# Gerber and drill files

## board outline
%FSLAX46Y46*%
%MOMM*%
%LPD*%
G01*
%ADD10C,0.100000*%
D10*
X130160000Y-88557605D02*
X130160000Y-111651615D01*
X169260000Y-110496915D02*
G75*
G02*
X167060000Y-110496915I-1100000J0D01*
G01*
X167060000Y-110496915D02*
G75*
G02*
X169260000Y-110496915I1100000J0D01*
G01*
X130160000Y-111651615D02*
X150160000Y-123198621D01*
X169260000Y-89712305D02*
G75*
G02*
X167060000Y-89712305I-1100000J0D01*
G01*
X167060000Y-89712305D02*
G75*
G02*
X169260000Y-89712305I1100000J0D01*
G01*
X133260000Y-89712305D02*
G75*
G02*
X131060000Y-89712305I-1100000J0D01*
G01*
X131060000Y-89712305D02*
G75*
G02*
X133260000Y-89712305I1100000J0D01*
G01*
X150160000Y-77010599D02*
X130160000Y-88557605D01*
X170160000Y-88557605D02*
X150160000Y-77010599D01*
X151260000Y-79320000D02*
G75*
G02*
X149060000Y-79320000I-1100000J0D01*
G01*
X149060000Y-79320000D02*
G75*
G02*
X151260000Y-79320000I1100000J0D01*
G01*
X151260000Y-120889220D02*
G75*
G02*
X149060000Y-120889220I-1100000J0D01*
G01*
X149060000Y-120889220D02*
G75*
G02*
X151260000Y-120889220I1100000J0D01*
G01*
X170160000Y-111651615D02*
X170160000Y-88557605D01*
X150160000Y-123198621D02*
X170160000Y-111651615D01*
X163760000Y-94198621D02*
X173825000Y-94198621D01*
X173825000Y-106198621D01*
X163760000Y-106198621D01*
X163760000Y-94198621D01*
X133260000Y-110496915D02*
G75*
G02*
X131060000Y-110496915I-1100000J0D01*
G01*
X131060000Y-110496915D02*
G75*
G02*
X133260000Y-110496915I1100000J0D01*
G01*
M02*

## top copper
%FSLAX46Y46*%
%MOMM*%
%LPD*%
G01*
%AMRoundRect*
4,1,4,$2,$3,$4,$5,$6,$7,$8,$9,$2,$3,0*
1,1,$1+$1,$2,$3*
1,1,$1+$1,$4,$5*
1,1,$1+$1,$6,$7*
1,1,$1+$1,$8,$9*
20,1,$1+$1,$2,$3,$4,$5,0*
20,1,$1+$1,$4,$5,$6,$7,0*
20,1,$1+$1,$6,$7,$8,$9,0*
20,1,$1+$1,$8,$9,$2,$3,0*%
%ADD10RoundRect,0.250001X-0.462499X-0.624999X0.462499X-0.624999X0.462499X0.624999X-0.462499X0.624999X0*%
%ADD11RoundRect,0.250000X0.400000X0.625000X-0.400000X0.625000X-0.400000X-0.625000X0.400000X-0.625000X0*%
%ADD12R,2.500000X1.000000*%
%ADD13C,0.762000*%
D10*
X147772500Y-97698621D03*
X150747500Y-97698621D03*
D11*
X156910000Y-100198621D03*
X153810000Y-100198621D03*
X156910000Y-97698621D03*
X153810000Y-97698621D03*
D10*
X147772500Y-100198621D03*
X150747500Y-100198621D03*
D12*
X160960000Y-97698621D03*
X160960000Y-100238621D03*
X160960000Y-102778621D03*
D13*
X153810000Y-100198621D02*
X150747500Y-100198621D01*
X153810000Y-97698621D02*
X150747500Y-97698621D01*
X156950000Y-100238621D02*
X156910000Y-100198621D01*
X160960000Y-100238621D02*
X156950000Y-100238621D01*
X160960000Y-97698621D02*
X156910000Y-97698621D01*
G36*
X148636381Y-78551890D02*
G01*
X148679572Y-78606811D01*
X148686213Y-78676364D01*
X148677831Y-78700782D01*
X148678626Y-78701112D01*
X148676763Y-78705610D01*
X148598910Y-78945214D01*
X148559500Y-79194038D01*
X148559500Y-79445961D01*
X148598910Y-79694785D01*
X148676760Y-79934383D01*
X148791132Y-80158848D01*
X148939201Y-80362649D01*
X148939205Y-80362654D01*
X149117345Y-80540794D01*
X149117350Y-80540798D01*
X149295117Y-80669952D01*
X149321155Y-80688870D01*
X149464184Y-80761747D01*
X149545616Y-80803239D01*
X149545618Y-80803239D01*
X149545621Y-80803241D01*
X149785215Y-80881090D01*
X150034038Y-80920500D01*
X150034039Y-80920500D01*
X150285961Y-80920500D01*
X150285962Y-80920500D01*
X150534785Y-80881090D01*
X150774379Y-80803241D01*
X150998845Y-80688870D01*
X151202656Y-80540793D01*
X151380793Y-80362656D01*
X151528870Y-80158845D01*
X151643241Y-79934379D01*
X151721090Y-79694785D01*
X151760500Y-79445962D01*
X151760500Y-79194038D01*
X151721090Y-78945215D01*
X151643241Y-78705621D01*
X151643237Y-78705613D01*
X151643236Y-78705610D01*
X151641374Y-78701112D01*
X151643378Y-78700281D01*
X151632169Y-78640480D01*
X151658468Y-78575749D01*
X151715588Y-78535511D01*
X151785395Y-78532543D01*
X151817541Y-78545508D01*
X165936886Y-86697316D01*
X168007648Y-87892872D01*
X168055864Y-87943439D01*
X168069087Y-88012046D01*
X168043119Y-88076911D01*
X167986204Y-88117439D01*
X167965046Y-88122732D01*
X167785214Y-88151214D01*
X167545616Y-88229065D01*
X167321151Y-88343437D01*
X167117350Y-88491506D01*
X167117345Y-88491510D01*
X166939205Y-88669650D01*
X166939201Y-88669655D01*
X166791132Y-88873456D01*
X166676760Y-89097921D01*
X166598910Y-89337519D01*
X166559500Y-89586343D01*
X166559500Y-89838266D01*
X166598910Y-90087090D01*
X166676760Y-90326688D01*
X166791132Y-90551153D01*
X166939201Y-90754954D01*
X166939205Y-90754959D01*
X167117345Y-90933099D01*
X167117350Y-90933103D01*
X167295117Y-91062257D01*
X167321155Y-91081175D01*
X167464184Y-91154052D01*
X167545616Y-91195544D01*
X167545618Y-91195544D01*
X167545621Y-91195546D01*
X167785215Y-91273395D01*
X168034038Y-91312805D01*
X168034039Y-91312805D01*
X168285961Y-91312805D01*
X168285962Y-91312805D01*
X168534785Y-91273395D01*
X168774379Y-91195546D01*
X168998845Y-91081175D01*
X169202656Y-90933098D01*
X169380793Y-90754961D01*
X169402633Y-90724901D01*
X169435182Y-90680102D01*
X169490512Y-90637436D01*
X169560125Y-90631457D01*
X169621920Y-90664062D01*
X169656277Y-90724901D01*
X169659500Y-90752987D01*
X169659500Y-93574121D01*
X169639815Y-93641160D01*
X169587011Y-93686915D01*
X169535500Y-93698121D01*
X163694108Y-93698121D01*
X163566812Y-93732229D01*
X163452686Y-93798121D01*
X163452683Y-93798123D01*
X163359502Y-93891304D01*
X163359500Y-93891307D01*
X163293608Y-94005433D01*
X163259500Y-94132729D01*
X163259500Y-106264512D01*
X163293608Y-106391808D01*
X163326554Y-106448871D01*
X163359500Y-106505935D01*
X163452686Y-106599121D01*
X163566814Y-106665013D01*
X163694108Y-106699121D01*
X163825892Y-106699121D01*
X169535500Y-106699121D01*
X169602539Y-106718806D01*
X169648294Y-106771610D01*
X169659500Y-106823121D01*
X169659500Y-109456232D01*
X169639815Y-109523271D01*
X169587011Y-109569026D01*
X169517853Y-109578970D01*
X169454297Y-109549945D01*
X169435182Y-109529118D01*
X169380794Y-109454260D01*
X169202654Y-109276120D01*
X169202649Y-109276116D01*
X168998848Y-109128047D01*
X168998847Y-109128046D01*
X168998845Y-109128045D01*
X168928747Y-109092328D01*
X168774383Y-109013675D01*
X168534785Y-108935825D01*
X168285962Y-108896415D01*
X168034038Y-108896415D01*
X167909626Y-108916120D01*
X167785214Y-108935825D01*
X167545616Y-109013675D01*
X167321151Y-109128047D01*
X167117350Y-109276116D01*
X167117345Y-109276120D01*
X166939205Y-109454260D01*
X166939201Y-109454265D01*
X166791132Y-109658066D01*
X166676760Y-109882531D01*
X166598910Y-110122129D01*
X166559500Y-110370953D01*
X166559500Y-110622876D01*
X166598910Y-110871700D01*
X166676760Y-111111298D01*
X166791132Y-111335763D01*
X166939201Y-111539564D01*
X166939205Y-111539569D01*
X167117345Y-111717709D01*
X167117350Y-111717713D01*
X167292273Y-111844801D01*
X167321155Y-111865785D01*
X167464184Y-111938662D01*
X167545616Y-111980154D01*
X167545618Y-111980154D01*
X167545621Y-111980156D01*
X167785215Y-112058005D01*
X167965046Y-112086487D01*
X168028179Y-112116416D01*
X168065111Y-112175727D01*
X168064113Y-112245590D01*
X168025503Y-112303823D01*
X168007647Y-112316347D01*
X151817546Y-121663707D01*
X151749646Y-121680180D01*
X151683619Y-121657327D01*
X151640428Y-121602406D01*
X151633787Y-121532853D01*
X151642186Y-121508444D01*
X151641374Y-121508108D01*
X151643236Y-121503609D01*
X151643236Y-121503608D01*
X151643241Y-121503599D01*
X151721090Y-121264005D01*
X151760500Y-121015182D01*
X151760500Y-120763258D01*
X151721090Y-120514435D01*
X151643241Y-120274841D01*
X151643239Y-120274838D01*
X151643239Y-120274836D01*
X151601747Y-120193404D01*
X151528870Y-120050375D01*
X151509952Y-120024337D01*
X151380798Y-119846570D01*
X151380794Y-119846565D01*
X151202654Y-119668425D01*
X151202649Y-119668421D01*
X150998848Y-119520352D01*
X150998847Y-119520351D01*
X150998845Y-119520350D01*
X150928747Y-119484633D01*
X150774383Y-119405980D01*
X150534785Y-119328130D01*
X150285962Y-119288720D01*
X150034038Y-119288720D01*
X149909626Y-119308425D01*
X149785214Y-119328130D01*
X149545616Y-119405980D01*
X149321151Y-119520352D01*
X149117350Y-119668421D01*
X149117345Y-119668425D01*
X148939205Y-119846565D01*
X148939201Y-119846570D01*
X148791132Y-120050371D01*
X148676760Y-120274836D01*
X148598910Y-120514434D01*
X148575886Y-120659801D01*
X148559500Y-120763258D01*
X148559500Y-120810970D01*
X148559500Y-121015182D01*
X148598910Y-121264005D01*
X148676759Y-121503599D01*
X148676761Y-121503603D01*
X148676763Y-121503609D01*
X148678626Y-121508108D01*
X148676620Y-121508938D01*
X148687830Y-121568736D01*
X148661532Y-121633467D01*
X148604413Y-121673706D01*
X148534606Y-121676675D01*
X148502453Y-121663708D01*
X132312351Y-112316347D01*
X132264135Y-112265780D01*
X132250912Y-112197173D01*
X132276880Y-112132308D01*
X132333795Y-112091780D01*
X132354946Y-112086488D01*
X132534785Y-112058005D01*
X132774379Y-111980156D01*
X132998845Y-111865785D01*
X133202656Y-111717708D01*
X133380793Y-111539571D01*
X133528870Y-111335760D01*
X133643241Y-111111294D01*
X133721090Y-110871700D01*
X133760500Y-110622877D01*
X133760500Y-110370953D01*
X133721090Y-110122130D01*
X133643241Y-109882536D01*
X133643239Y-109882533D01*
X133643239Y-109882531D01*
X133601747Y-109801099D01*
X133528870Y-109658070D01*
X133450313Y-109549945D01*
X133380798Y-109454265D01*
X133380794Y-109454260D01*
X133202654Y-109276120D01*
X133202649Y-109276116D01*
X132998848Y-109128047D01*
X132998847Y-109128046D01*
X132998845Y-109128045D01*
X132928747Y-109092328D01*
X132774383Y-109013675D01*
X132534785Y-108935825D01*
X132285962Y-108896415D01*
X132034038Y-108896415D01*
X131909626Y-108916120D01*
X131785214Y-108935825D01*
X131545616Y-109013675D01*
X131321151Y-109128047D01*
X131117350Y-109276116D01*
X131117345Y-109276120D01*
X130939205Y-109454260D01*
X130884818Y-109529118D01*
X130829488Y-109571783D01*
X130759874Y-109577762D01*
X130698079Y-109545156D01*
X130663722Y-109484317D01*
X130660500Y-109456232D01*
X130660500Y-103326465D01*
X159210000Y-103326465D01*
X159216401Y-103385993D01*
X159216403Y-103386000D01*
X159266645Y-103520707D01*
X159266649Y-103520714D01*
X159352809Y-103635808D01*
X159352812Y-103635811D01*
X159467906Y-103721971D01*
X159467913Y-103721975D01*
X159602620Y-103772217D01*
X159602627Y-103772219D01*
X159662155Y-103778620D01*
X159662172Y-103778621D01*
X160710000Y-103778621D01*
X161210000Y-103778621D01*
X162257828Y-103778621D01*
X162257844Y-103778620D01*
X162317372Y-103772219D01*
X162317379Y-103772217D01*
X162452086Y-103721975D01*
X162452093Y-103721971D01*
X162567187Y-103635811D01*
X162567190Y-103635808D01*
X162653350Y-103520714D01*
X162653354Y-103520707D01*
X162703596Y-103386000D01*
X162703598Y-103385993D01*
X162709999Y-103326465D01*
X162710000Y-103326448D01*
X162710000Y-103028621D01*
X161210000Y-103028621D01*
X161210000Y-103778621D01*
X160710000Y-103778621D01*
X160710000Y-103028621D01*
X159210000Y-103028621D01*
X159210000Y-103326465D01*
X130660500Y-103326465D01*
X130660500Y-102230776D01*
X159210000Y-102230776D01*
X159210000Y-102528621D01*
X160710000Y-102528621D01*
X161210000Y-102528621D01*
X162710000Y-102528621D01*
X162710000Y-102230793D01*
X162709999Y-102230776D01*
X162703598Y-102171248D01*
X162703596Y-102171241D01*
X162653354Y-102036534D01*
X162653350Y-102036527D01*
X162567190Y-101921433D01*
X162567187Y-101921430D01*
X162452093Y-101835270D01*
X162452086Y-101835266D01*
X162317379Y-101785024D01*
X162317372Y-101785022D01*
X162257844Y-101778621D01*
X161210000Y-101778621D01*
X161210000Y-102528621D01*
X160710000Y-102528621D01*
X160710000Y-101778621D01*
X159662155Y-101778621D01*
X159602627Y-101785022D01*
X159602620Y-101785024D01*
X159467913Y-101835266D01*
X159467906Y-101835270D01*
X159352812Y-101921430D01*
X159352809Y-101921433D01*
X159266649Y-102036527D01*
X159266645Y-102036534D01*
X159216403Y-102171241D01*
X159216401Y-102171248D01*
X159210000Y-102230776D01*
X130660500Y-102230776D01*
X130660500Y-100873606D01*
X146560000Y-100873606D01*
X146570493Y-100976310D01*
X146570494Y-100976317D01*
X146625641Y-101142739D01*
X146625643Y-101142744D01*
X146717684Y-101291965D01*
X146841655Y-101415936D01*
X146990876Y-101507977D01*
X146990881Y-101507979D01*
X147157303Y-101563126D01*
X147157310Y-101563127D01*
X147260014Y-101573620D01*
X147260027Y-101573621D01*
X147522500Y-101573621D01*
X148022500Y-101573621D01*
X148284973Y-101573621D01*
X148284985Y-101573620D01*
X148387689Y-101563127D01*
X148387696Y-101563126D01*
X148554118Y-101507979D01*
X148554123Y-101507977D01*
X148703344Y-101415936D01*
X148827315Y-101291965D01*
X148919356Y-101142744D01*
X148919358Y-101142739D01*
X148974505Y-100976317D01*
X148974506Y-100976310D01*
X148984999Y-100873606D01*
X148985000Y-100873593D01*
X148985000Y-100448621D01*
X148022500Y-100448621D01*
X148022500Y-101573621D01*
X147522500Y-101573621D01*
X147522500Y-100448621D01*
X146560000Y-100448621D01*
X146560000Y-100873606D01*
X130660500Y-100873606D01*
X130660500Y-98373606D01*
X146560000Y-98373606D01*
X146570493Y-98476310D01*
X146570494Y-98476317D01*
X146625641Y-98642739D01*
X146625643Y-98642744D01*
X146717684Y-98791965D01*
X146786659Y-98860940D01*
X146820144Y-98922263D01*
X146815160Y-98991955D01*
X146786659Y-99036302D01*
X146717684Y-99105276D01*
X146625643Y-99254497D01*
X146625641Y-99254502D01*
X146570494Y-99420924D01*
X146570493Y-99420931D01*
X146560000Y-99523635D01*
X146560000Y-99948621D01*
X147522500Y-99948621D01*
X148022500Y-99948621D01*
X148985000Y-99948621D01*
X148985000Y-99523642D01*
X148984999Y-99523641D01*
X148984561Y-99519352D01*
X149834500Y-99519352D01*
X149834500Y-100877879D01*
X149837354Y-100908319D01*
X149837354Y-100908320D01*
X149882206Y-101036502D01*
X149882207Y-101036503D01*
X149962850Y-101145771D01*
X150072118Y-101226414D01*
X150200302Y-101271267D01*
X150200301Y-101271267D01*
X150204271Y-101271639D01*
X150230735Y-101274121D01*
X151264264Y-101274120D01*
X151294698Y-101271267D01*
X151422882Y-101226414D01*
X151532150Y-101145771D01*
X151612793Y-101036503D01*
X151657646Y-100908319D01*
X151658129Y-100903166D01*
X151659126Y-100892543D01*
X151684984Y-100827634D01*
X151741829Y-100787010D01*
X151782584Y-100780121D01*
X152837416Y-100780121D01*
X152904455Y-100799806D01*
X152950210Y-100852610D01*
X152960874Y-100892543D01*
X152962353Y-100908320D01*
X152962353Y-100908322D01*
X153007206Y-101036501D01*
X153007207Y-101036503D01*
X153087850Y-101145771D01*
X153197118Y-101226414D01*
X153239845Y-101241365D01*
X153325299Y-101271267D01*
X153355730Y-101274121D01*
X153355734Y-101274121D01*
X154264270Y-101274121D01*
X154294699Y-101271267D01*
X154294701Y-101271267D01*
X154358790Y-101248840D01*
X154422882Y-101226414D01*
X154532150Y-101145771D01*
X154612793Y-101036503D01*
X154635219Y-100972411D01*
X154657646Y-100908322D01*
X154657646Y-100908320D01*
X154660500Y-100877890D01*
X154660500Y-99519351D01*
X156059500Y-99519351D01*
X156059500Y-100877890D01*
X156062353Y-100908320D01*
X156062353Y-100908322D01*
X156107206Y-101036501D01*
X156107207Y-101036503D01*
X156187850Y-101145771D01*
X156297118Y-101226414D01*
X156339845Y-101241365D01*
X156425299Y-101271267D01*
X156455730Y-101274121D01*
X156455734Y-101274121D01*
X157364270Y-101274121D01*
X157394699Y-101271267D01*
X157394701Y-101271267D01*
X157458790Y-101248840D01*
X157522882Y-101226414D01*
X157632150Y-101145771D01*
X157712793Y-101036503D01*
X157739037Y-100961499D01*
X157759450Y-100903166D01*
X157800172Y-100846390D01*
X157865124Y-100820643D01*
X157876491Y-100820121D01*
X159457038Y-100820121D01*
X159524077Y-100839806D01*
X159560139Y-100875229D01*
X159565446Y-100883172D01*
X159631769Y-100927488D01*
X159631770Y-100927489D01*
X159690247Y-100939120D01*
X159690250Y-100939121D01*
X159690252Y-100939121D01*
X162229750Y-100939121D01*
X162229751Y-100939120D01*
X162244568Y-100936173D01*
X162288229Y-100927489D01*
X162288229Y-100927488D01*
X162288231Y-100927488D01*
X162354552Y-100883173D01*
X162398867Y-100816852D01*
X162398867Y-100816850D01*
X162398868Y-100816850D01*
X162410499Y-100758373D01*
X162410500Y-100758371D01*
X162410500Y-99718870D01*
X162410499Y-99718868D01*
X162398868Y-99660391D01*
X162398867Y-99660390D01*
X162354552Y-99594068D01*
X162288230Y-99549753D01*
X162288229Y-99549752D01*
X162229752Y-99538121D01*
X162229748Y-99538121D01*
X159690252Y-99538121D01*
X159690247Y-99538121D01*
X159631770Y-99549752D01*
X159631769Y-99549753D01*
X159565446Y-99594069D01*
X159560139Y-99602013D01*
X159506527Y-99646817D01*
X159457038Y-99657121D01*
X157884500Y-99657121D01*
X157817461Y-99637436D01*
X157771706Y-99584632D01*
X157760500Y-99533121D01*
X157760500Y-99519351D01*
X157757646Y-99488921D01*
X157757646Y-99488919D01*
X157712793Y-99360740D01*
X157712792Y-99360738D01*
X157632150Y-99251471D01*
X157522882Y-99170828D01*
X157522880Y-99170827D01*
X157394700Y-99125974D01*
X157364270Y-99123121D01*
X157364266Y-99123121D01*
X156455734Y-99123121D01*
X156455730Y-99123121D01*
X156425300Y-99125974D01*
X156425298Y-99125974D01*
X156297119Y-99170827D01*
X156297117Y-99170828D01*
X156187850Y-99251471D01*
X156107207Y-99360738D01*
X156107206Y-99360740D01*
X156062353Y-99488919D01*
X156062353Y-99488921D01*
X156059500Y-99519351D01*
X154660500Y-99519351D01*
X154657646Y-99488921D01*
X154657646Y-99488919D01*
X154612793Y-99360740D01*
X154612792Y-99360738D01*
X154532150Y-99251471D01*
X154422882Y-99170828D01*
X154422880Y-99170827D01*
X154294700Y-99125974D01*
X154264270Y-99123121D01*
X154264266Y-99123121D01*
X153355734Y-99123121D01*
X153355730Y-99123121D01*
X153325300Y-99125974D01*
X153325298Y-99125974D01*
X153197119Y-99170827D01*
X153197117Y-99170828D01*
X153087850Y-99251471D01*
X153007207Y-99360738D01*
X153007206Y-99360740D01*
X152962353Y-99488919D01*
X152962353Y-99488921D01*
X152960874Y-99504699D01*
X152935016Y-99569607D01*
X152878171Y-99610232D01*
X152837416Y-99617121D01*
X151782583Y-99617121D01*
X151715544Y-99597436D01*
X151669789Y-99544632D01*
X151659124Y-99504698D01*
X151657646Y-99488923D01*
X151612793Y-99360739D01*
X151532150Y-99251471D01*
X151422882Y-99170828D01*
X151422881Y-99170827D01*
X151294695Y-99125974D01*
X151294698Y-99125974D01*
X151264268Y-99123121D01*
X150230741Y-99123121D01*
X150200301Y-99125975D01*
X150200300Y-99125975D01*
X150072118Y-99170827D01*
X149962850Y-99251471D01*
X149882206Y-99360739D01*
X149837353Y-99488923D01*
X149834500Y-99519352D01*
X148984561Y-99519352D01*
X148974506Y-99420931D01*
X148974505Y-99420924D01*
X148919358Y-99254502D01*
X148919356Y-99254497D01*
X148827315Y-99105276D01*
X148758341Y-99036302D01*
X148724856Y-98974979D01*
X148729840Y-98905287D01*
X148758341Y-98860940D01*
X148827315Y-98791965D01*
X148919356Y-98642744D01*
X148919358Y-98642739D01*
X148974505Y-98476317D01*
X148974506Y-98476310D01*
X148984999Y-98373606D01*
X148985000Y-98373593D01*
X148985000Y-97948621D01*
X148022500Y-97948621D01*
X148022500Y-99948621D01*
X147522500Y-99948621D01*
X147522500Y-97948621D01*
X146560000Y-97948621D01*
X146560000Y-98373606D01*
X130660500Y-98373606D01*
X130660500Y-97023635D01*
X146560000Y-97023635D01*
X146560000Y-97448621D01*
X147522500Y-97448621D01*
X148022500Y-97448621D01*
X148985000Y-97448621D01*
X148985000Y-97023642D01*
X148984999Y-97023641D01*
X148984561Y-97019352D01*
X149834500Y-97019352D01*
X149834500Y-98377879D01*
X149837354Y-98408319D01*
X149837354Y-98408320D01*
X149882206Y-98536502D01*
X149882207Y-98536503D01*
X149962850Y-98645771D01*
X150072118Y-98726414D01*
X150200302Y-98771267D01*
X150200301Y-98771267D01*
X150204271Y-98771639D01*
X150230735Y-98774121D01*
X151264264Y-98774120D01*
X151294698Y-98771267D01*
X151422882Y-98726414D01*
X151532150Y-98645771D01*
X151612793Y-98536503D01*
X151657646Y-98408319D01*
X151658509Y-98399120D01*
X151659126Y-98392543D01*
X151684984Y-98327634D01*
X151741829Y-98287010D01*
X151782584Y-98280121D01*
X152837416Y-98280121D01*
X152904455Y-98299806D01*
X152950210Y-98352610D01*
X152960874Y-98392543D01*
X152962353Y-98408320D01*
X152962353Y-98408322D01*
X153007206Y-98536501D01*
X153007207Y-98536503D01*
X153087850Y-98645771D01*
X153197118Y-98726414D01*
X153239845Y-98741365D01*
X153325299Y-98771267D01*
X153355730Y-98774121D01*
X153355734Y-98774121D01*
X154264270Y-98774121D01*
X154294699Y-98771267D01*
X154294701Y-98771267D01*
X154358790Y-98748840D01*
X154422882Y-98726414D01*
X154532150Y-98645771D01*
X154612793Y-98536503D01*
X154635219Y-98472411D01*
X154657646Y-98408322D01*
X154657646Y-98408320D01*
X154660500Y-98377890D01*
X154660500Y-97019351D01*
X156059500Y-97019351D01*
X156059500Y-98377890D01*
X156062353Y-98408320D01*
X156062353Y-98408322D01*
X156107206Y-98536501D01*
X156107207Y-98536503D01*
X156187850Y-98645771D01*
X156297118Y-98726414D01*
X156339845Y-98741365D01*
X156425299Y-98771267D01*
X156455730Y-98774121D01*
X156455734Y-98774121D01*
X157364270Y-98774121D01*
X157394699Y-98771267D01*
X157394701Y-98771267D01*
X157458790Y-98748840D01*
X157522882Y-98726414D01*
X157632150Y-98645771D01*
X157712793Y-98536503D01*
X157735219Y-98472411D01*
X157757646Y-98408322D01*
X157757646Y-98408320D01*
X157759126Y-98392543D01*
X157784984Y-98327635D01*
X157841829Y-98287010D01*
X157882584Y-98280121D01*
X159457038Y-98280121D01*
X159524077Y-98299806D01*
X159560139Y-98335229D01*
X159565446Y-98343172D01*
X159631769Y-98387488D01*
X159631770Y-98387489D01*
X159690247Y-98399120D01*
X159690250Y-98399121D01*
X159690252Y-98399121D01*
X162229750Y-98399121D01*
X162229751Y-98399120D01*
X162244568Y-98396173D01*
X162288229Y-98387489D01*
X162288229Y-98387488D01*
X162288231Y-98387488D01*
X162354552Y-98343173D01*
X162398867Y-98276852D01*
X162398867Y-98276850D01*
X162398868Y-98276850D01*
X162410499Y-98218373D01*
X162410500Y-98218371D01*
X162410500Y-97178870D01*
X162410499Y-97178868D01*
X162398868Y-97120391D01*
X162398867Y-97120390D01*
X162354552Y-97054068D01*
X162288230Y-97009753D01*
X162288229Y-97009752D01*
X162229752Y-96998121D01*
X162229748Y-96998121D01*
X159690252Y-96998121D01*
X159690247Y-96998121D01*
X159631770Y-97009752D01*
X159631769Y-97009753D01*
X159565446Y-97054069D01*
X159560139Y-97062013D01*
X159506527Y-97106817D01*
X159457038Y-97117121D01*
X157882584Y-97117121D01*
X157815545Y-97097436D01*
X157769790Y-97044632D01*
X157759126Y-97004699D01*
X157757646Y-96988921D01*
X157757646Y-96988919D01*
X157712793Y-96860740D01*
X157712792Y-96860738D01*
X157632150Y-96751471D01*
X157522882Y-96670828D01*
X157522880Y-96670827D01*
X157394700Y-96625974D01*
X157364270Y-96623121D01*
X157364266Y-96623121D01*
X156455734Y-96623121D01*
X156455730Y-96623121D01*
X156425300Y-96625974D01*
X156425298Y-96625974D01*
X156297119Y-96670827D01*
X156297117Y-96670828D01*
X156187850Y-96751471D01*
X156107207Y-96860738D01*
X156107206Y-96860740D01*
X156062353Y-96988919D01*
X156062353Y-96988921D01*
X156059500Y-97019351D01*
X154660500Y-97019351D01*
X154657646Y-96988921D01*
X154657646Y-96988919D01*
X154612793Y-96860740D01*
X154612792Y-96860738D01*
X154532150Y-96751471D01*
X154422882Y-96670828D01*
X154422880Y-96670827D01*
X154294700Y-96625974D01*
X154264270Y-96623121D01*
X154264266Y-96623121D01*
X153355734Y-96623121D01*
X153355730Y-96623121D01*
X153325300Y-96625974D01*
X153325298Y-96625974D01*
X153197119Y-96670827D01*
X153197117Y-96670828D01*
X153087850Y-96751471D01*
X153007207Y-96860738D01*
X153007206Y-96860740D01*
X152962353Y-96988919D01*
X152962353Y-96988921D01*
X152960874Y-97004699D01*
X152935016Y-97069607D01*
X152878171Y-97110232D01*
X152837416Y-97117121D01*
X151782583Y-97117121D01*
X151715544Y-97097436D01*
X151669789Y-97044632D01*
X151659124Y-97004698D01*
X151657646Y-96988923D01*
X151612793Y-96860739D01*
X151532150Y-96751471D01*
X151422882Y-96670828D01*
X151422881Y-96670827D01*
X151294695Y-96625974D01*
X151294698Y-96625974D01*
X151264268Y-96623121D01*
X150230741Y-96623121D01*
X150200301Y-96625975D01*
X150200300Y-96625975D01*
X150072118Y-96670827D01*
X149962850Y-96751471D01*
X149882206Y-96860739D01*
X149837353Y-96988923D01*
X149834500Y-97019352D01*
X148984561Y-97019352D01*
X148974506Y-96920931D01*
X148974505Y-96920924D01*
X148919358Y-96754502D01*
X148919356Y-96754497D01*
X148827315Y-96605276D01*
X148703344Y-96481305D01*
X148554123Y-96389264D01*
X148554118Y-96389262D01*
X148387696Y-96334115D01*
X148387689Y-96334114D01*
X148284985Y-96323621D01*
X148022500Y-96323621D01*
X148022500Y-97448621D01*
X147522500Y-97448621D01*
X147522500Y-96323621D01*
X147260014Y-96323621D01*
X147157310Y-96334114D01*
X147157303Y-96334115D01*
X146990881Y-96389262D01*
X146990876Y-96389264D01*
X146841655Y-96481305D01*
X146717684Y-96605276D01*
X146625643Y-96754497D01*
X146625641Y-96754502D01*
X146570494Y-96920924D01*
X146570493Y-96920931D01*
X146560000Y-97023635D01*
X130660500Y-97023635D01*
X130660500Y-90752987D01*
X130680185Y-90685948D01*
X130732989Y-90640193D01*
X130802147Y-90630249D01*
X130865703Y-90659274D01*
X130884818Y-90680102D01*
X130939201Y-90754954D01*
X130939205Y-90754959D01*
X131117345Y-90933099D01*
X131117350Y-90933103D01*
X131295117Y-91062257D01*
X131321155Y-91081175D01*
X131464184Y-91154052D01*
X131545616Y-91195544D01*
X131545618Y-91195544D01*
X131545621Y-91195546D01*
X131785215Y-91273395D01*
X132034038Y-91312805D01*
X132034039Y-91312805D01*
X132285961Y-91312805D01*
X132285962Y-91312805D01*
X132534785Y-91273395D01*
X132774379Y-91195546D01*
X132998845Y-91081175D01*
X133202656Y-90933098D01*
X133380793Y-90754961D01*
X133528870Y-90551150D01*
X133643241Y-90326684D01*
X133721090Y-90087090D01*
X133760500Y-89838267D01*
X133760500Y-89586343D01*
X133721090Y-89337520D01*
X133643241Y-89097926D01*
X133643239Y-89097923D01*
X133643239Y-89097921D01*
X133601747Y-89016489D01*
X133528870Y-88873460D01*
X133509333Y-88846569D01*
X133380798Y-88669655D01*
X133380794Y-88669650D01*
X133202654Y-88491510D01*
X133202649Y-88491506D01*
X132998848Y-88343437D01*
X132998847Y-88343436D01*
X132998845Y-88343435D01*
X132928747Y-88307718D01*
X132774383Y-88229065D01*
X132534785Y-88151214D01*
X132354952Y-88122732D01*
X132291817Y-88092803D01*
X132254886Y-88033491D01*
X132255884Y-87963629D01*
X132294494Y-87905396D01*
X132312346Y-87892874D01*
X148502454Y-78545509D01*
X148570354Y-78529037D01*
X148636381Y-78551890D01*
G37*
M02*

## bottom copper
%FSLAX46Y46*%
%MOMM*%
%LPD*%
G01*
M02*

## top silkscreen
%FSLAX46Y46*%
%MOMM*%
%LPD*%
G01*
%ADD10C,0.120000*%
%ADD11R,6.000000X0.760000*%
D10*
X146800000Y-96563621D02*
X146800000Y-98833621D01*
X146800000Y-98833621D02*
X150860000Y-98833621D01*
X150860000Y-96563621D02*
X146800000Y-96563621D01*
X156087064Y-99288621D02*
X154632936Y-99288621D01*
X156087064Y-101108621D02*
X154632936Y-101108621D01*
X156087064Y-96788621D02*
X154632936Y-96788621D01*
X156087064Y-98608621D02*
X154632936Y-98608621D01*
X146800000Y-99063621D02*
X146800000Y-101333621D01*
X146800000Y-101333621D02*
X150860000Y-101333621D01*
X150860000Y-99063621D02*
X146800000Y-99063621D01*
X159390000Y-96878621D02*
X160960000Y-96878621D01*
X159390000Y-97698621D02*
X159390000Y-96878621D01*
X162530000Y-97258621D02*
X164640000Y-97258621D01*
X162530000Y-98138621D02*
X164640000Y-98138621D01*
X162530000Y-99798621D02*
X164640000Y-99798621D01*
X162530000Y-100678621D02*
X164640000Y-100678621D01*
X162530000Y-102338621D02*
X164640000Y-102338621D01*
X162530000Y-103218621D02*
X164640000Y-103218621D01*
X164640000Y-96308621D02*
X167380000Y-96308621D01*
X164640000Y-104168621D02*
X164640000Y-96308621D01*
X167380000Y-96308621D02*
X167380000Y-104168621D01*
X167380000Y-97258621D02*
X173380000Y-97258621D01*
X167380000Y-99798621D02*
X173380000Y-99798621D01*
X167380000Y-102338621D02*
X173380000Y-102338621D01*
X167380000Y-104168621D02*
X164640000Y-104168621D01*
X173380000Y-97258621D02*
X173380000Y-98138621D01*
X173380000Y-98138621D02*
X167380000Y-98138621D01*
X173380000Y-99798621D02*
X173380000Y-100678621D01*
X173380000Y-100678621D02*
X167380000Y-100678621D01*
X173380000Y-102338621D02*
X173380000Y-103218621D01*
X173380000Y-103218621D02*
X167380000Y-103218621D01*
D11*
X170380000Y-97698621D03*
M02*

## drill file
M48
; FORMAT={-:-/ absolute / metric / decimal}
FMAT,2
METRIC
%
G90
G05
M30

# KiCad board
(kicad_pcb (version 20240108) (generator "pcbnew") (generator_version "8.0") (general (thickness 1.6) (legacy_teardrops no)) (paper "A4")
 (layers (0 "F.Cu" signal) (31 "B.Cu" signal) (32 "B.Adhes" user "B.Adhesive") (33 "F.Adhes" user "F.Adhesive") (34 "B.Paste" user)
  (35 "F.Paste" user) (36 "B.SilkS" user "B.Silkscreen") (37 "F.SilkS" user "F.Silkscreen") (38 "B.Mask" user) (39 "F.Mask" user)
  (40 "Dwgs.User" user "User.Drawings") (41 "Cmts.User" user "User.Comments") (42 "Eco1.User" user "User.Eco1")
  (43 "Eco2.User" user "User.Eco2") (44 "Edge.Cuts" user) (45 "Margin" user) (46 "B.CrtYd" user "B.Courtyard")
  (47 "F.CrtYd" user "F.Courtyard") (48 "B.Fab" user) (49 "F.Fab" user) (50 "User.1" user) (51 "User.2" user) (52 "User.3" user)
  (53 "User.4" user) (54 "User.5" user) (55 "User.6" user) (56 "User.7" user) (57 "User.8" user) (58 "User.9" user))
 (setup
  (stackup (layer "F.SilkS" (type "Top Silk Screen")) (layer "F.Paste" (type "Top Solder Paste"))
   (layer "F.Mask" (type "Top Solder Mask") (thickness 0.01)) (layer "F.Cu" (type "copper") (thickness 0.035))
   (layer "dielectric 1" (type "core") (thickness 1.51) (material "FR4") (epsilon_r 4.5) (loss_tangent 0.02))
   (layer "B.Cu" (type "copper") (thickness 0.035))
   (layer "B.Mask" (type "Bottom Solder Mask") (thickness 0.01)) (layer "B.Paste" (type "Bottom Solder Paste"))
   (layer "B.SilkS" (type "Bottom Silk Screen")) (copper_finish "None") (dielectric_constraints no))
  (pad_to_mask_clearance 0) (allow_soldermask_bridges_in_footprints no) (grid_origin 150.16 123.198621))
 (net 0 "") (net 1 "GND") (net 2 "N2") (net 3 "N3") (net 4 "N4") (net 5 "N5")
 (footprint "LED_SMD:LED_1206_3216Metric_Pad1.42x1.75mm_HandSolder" (layer "F.Cu") (at 149.26 97.698621)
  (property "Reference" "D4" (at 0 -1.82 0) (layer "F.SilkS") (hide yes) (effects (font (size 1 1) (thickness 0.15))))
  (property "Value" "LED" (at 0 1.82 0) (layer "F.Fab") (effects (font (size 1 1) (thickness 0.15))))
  (fp_line (start -2.46 -1.135) (end -2.46 1.135) (stroke (width 0.12) (type solid)) (layer "F.SilkS"))
  (fp_line (start -2.46 1.135) (end 1.6 1.135) (stroke (width 0.12) (type solid)) (layer "F.SilkS"))
  (fp_line (start 1.6 -1.135) (end -2.46 -1.135) (stroke (width 0.12) (type solid)) (layer "F.SilkS"))
  (pad "1" smd roundrect (at -1.4875 0) (size 1.425 1.75) (layers "F.Cu" "F.Paste" "F.Mask") (roundrect_rratio 0.175439) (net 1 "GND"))
  (pad "2" smd roundrect (at 1.4875 0) (size 1.425 1.75) (layers "F.Cu" "F.Paste" "F.Mask") (roundrect_rratio 0.175439) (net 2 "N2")))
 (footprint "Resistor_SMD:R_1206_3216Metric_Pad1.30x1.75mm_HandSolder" (layer "F.Cu") (at 155.36 100.198621 180)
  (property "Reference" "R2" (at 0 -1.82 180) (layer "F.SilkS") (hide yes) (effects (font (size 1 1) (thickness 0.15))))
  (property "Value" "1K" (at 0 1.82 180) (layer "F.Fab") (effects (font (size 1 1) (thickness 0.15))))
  (fp_line (start -0.727064 0.91) (end 0.727064 0.91) (stroke (width 0.12) (type solid)) (layer "F.SilkS"))
  (fp_line (start -0.727064 -0.91) (end 0.727064 -0.91) (stroke (width 0.12) (type solid)) (layer "F.SilkS"))
  (pad "1" smd roundrect (at -1.55 0 180) (size 1.3 1.75) (layers "F.Cu" "F.Paste" "F.Mask") (roundrect_rratio 0.192308) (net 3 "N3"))
  (pad "2" smd roundrect (at 1.55 0 180) (size 1.3 1.75) (layers "F.Cu" "F.Paste" "F.Mask") (roundrect_rratio 0.192308) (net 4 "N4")))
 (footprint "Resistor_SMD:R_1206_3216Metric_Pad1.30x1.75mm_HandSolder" (layer "F.Cu") (at 155.36 97.698621 180)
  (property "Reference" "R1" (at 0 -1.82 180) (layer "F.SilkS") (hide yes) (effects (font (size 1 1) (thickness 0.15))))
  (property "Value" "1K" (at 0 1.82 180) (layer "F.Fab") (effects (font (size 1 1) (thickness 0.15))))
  (fp_line (start -0.727064 0.91) (end 0.727064 0.91) (stroke (width 0.12) (type solid)) (layer "F.SilkS"))
  (fp_line (start -0.727064 -0.91) (end 0.727064 -0.91) (stroke (width 0.12) (type solid)) (layer "F.SilkS"))
  (pad "1" smd roundrect (at -1.55 0 180) (size 1.3 1.75) (layers "F.Cu" "F.Paste" "F.Mask") (roundrect_rratio 0.192308) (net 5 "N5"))
  (pad "2" smd roundrect (at 1.55 0 180) (size 1.3 1.75) (layers "F.Cu" "F.Paste" "F.Mask") (roundrect_rratio 0.192308) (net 2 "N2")))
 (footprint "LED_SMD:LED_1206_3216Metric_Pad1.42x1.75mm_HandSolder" (layer "F.Cu") (at 149.26 100.198621)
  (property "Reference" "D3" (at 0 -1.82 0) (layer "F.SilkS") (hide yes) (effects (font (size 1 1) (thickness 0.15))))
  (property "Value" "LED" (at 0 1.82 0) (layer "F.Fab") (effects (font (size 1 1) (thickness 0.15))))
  (fp_line (start -2.46 -1.135) (end -2.46 1.135) (stroke (width 0.12) (type solid)) (layer "F.SilkS"))
  (fp_line (start -2.46 1.135) (end 1.6 1.135) (stroke (width 0.12) (type solid)) (layer "F.SilkS"))
  (fp_line (start 1.6 -1.135) (end -2.46 -1.135) (stroke (width 0.12) (type solid)) (layer "F.SilkS"))
  (pad "1" smd roundrect (at -1.4875 0) (size 1.425 1.75) (layers "F.Cu" "F.Paste" "F.Mask") (roundrect_rratio 0.175439) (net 1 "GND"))
  (pad "2" smd roundrect (at 1.4875 0) (size 1.425 1.75) (layers "F.Cu" "F.Paste" "F.Mask") (roundrect_rratio 0.175439) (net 4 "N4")))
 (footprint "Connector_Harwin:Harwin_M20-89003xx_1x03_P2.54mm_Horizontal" (layer "F.Cu") (at 166.485 100.238621)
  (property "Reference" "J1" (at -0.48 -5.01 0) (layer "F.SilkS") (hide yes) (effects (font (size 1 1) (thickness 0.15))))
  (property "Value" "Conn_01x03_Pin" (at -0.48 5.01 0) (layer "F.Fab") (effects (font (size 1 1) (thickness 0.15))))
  (fp_line (start -7.095 -3.36) (end -5.525 -3.36) (stroke (width 0.12) (type solid)) (layer "F.SilkS"))
  (fp_line (start -7.095 -2.54) (end -7.095 -3.36) (stroke (width 0.12) (type solid)) (layer "F.SilkS"))
  (fp_line (start -3.955 -2.98) (end -1.845 -2.98) (stroke (width 0.12) (type solid)) (layer "F.SilkS"))
  (fp_line (start -3.955 -2.1) (end -1.845 -2.1) (stroke (width 0.12) (type solid)) (layer "F.SilkS"))
  (fp_line (start -3.955 -0.44) (end -1.845 -0.44) (stroke (width 0.12) (type solid)) (layer "F.SilkS"))
  (fp_line (start -3.955 0.44) (end -1.845 0.44) (stroke (width 0.12) (type solid)) (layer "F.SilkS"))
  (fp_line (start -3.955 2.1) (end -1.845 2.1) (stroke (width 0.12) (type solid)) (layer "F.SilkS"))
  (fp_line (start -3.955 2.98) (end -1.845 2.98) (stroke (width 0.12) (type solid)) (layer "F.SilkS"))
  (fp_line (start -1.845 -3.93) (end 0.895 -3.93) (stroke (width 0.12) (type solid)) (layer "F.SilkS"))
  (fp_line (start -1.845 3.93) (end -1.845 -3.93) (stroke (width 0.12) (type solid)) (layer "F.SilkS"))
  (fp_line (start 0.895 -3.93) (end 0.895 3.93) (stroke (width 0.12) (type solid)) (layer "F.SilkS"))
  (fp_line (start 0.895 -2.98) (end 6.895 -2.98) (stroke (width 0.12) (type solid)) (layer "F.SilkS"))
  (fp_line (start 0.895 -0.44) (end 6.895 -0.44) (stroke (width 0.12) (type solid)) (layer "F.SilkS"))
  (fp_line (start 0.895 2.1) (end 6.895 2.1) (stroke (width 0.12) (type solid)) (layer "F.SilkS"))
  (fp_line (start 0.895 3.93) (end -1.845 3.93) (stroke (width 0.12) (type solid)) (layer "F.SilkS"))
  (fp_line (start 6.895 -2.98) (end 6.895 -2.1) (stroke (width 0.12) (type solid)) (layer "F.SilkS"))
  (fp_line (start 6.895 -2.1) (end 0.895 -2.1) (stroke (width 0.12) (type solid)) (layer "F.SilkS"))
  (fp_line (start 6.895 -0.44) (end 6.895 0.44) (stroke (width 0.12) (type solid)) (layer "F.SilkS"))
  (fp_line (start 6.895 0.44) (end 0.895 0.44) (stroke (width 0.12) (type solid)) (layer "F.SilkS"))
  (fp_line (start 6.895 2.1) (end 6.895 2.98) (stroke (width 0.12) (type solid)) (layer "F.SilkS"))
  (fp_line (start 6.895 2.98) (end 0.895 2.98) (stroke (width 0.12) (type solid)) (layer "F.SilkS"))
  (pad "" smd rect (at 3.895 -2.54) (size 6 0.76) (layers "F.SilkS"))
  (pad "1" smd rect (at -5.525 -2.54) (size 2.5 1) (layers "F.Cu" "F.Paste" "F.Mask") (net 5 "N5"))
  (pad "2" smd rect (at -5.525 0) (size 2.5 1) (layers "F.Cu" "F.Paste" "F.Mask") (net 3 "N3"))
  (pad "3" smd rect (at -5.525 2.54) (size 2.5 1) (layers "F.Cu" "F.Paste" "F.Mask") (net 1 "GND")))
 (gr_line (start 130.16 88.557605) (end 130.16 111.651615) (stroke (width 0.1) (type solid)) (layer "Edge.Cuts"))
 (gr_circle (center 168.16 110.496915) (end 169.26 110.496915) (stroke (width 0.1) (type solid)) (fill none) (layer "Edge.Cuts"))
 (gr_line (start 130.16 111.651615) (end 150.16 123.198621) (stroke (width 0.1) (type solid)) (layer "Edge.Cuts"))
 (gr_circle (center 168.16 89.712305) (end 169.26 89.712305) (stroke (width 0.1) (type solid)) (fill none) (layer "Edge.Cuts"))
 (gr_circle (center 132.16 89.712305) (end 133.26 89.712305) (stroke (width 0.1) (type solid)) (fill none) (layer "Edge.Cuts"))
 (gr_line (start 150.16 77.010599) (end 130.16 88.557605) (stroke (width 0.1) (type solid)) (layer "Edge.Cuts"))
 (gr_line (start 170.16 88.557605) (end 150.16 77.010599) (stroke (width 0.1) (type solid)) (layer "Edge.Cuts"))
 (gr_circle (center 150.16 79.32) (end 151.26 79.32) (stroke (width 0.1) (type solid)) (fill none) (layer "Edge.Cuts"))
 (gr_circle (center 150.16 120.88922) (end 151.26 120.88922) (stroke (width 0.1) (type solid)) (fill none) (layer "Edge.Cuts"))
 (gr_line (start 170.16 111.651615) (end 170.16 88.557605) (stroke (width 0.1) (type solid)) (layer "Edge.Cuts"))
 (gr_line (start 150.16 123.198621) (end 170.16 111.651615) (stroke (width 0.1) (type solid)) (layer "Edge.Cuts"))
 (gr_rect (start 163.76 94.198621) (end 173.825 106.198621) (stroke (width 0.1) (type default)) (fill none) (layer "Edge.Cuts"))
 (gr_circle (center 132.16 110.496915) (end 133.26 110.496915) (stroke (width 0.1) (type solid)) (fill none) (layer "Edge.Cuts"))
 (segment (start 153.81 100.198621) (end 150.7475 100.198621) (width 0.762) (layer "F.Cu") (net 4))
 (segment (start 153.81 97.698621) (end 150.7475 97.698621) (width 0.762) (layer "F.Cu") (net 2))
 (segment (start 156.95 100.238621) (end 156.91 100.198621) (width 0.762) (layer "F.Cu") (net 3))
 (segment (start 160.96 100.238621) (end 156.95 100.238621) (width 0.762) (layer "F.Cu") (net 3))
 (segment (start 160.96 97.698621) (end 156.91 97.698621) (width 0.762) (layer "F.Cu") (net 5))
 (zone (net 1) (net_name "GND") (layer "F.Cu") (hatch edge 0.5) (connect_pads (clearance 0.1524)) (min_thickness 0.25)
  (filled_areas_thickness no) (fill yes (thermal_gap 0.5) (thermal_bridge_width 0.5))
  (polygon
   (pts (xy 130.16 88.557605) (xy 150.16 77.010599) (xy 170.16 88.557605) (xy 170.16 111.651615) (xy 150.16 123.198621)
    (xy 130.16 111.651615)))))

